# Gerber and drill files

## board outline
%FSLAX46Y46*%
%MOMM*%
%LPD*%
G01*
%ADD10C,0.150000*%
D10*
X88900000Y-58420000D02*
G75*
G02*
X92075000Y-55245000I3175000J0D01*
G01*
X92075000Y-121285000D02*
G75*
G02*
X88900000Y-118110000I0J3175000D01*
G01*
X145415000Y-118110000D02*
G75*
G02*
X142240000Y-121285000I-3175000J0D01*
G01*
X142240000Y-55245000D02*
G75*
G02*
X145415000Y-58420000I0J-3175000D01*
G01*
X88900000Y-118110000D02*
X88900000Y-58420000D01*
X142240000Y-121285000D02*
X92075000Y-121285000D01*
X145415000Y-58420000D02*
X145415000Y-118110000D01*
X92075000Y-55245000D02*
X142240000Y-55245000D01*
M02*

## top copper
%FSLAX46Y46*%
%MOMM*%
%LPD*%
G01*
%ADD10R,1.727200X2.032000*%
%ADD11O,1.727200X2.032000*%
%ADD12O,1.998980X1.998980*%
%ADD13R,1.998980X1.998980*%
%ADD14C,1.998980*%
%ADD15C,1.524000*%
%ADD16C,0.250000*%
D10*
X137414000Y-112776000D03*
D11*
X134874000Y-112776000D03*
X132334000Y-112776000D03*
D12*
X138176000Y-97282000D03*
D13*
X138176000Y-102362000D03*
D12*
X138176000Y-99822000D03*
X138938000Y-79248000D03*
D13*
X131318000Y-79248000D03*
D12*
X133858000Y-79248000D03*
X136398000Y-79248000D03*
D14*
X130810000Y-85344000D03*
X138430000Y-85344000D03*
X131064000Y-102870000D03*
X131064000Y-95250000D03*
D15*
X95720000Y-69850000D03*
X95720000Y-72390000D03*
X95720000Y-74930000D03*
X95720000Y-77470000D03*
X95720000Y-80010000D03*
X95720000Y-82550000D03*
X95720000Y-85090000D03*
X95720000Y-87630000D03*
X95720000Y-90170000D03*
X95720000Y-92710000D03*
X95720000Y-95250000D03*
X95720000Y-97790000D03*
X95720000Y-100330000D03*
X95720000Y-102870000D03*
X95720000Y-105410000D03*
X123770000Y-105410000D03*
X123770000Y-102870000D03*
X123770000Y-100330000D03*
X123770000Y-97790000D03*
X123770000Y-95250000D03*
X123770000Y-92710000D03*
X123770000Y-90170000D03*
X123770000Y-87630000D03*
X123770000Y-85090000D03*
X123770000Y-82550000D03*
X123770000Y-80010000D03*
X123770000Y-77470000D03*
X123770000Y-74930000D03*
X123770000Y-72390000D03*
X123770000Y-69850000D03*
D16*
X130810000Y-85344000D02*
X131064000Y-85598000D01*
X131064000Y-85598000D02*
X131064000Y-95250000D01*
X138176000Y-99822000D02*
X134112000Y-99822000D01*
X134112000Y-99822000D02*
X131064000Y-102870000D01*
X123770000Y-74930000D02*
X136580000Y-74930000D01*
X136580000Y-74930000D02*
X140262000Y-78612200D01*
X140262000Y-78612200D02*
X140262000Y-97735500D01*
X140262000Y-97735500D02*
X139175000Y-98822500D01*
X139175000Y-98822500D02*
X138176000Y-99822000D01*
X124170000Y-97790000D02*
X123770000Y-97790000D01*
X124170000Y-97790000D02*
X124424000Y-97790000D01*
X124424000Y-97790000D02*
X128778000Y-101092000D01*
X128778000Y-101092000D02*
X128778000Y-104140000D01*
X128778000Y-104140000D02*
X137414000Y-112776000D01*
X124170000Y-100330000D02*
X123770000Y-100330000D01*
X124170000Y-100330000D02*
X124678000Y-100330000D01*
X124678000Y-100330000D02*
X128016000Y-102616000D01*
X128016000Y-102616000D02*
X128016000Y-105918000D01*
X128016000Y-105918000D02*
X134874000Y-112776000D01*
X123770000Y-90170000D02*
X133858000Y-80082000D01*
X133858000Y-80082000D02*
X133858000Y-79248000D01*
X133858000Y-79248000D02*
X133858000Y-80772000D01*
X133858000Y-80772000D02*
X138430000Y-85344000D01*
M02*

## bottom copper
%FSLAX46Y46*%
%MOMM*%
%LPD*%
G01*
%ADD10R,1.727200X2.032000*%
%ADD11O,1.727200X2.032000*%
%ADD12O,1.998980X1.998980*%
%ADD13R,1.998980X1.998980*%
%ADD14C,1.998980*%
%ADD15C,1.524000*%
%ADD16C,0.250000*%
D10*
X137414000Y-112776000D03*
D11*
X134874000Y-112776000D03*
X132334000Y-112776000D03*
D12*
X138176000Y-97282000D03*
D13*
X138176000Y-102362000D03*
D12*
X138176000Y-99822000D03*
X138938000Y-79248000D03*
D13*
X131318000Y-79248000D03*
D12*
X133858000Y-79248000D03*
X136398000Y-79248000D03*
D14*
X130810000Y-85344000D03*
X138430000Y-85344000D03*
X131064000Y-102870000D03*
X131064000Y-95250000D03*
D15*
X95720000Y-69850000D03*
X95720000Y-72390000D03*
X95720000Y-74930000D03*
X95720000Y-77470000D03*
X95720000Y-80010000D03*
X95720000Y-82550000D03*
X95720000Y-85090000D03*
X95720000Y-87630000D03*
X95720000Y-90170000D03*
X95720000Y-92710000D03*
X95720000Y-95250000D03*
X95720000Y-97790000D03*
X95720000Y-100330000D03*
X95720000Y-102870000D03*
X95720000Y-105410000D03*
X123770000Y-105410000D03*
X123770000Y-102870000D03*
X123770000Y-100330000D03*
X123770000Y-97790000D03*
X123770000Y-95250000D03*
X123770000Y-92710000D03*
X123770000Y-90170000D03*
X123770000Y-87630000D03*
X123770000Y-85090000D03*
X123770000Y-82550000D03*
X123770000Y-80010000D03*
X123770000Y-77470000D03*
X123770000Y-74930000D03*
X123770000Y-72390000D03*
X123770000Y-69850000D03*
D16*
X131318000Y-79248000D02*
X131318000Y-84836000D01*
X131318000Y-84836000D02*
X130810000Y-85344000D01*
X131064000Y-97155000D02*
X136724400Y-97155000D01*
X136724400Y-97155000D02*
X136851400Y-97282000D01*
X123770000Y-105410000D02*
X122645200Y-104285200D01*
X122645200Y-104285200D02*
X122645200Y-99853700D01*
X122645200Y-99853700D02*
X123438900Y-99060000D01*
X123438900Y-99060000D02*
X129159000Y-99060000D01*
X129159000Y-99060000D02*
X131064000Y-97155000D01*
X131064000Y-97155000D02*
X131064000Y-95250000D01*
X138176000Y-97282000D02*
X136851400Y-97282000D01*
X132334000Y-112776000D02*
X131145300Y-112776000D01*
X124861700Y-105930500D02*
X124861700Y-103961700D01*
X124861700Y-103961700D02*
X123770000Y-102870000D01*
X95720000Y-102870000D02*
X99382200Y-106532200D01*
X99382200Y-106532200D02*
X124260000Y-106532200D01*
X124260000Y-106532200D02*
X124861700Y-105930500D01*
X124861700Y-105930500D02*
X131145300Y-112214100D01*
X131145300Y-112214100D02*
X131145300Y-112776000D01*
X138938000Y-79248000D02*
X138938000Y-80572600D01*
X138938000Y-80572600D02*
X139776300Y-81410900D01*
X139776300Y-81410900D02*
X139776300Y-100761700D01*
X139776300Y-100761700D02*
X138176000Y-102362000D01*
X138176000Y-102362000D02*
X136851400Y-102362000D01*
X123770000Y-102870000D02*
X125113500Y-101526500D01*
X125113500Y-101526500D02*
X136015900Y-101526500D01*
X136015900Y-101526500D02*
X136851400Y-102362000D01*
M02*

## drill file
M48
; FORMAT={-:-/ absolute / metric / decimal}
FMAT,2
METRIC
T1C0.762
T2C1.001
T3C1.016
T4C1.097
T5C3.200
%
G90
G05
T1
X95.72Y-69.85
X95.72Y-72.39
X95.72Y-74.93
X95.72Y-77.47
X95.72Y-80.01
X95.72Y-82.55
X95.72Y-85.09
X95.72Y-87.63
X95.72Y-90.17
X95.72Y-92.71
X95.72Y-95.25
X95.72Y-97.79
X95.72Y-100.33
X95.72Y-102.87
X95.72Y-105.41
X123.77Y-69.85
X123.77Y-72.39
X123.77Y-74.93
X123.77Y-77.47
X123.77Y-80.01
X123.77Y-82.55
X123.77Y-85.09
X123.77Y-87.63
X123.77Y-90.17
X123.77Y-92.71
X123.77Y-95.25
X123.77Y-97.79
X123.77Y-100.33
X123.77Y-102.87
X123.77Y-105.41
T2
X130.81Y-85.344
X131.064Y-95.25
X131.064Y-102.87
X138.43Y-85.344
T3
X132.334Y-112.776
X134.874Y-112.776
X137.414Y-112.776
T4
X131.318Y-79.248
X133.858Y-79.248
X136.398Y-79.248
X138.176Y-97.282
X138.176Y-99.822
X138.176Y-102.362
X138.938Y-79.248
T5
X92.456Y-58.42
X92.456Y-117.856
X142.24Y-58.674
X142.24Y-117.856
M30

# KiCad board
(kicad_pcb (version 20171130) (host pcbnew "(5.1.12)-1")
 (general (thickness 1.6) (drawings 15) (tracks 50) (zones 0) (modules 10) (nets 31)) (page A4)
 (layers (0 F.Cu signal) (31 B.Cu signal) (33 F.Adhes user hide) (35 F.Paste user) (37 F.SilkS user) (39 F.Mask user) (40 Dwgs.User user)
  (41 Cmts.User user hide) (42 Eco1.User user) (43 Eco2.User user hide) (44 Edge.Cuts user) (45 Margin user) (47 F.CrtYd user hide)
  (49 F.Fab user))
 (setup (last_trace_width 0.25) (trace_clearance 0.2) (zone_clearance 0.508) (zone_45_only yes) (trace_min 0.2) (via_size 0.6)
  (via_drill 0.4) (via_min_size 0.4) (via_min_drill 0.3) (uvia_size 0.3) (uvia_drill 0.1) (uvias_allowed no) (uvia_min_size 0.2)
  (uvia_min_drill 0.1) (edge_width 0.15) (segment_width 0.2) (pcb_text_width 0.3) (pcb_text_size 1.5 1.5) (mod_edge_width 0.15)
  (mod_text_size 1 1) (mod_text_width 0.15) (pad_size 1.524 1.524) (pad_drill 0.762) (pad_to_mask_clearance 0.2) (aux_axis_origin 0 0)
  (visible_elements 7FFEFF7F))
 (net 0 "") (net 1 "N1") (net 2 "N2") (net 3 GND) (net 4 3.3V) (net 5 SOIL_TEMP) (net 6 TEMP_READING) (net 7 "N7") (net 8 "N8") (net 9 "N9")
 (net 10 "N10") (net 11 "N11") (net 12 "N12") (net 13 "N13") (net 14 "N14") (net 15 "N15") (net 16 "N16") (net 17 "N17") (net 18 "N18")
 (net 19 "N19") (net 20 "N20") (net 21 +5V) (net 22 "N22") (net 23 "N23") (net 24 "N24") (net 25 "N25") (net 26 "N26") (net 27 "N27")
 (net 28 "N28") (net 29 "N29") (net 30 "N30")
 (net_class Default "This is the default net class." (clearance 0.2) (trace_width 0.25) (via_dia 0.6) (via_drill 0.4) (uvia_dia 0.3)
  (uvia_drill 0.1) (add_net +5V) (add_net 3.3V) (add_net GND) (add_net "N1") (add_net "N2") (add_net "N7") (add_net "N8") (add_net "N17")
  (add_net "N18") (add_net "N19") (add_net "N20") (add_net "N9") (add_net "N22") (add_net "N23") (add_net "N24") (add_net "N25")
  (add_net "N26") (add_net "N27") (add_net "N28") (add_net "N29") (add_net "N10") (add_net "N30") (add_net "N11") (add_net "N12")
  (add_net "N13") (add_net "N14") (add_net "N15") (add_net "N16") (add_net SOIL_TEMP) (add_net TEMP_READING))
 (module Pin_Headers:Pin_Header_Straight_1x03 (layer F.Cu) (at 137.414 112.776 270)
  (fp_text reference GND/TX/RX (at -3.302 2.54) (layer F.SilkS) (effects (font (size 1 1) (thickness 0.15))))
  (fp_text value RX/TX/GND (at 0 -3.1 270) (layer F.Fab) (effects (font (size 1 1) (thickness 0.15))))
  (pad 1 thru_hole rect (at 0 0 270) (size 2.032 1.7272) (drill 1.016) (layers *.Cu *.Mask F.SilkS) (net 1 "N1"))
  (pad 2 thru_hole oval (at 0 2.54 270) (size 2.032 1.7272) (drill 1.016) (layers *.Cu *.Mask F.SilkS) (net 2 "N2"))
  (pad 3 thru_hole oval (at 0 5.08 270) (size 2.032 1.7272) (drill 1.016) (layers *.Cu *.Mask F.SilkS) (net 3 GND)))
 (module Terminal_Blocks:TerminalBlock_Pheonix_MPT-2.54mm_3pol (layer F.Cu) (at 138.176 102.362 90)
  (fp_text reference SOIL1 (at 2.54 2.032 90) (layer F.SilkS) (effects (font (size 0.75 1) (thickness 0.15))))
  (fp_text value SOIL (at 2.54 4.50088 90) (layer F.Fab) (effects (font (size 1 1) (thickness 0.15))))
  (pad 3 thru_hole oval (at 5.08 0 90) (size 1.99898 1.99898) (drill 1.09728) (layers *.Cu *.Mask F.SilkS) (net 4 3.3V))
  (pad 1 thru_hole rect (at 0 0 90) (size 1.99898 1.99898) (drill 1.09728) (layers *.Cu *.Mask F.SilkS) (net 3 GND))
  (pad 2 thru_hole oval (at 2.54 0 90) (size 1.99898 1.99898) (drill 1.09728) (layers *.Cu *.Mask F.SilkS) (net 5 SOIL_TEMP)))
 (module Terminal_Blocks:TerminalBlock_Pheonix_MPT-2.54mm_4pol (layer F.Cu) (at 131.318 79.248)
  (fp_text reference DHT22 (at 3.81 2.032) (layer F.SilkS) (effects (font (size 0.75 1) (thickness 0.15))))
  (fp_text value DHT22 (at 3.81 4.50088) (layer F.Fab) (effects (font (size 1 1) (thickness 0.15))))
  (pad 4 thru_hole oval (at 7.62 0 180) (size 1.99898 1.99898) (drill 1.09728) (layers *.Cu *.Mask F.SilkS) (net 3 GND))
  (pad 1 thru_hole rect (at 0 0 180) (size 1.99898 1.99898) (drill 1.09728) (layers *.Cu *.Mask F.SilkS) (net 4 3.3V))
  (pad 2 thru_hole oval (at 2.54 0 180) (size 1.99898 1.99898) (drill 1.09728) (layers *.Cu *.Mask F.SilkS) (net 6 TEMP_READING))
  (pad 3 thru_hole oval (at 5.08 0 180) (size 1.99898 1.99898) (drill 1.09728) (layers *.Cu *.Mask F.SilkS) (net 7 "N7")))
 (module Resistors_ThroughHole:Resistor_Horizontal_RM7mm (layer F.Cu) (at 130.81 85.344)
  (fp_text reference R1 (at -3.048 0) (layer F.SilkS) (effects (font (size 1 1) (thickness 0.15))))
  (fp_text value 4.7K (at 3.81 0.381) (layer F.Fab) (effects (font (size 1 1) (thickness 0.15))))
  (pad 1 thru_hole circle (at 0 0) (size 1.99898 1.99898) (drill 1.00076) (layers *.Cu *.SilkS *.Mask) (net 4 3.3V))
  (pad 2 thru_hole circle (at 7.62 0) (size 1.99898 1.99898) (drill 1.00076) (layers *.Cu *.SilkS *.Mask) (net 6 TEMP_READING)))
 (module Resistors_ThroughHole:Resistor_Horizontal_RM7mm (layer F.Cu) (at 131.064 102.87 90)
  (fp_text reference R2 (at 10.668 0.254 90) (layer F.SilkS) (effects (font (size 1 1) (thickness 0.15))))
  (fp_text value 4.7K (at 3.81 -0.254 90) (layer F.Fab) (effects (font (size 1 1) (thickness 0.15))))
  (pad 1 thru_hole circle (at 0 0 90) (size 1.99898 1.99898) (drill 1.00076) (layers *.Cu *.SilkS *.Mask) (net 5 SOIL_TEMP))
  (pad 2 thru_hole circle (at 7.62 0 90) (size 1.99898 1.99898) (drill 1.00076) (layers *.Cu *.SilkS *.Mask) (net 4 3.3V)))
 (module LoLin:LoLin (layer F.Cu) (at 93.98 59.69)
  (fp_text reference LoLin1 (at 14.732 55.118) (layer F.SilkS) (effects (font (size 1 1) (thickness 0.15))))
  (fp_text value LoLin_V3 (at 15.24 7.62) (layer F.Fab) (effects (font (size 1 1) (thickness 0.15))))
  (pad 1 thru_hole circle (at 1.74 10.16) (size 1.524 1.524) (drill 0.762) (layers *.Cu *.Mask F.SilkS) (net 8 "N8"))
  (pad 2 thru_hole circle (at 1.74 12.7) (size 1.524 1.524) (drill 0.762) (layers *.Cu *.Mask F.SilkS) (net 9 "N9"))
  (pad 3 thru_hole circle (at 1.74 15.24) (size 1.524 1.524) (drill 0.762) (layers *.Cu *.Mask F.SilkS) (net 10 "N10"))
  (pad 4 thru_hole circle (at 1.74 17.78) (size 1.524 1.524) (drill 0.762) (layers *.Cu *.Mask F.SilkS) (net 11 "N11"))
  (pad 5 thru_hole circle (at 1.74 20.32) (size 1.524 1.524) (drill 0.762) (layers *.Cu *.Mask F.SilkS) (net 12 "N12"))
  (pad 6 thru_hole circle (at 1.74 22.86) (size 1.524 1.524) (drill 0.762) (layers *.Cu *.Mask F.SilkS) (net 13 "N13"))
  (pad 7 thru_hole circle (at 1.74 25.4) (size 1.524 1.524) (drill 0.762) (layers *.Cu *.Mask F.SilkS) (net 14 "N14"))
  (pad 8 thru_hole circle (at 1.74 27.94) (size 1.524 1.524) (drill 0.762) (layers *.Cu *.Mask F.SilkS) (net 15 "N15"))
  (pad 9 thru_hole circle (at 1.74 30.48) (size 1.524 1.524) (drill 0.762) (layers *.Cu *.Mask F.SilkS) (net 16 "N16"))
  (pad 10 thru_hole circle (at 1.74 33.02) (size 1.524 1.524) (drill 0.762) (layers *.Cu *.Mask F.SilkS) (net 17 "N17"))
  (pad 11 thru_hole circle (at 1.74 35.56) (size 1.524 1.524) (drill 0.762) (layers *.Cu *.Mask F.SilkS) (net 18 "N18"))
  (pad 12 thru_hole circle (at 1.74 38.1) (size 1.524 1.524) (drill 0.762) (layers *.Cu *.Mask F.SilkS) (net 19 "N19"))
  (pad 13 thru_hole circle (at 1.74 40.64) (size 1.524 1.524) (drill 0.762) (layers *.Cu *.Mask F.SilkS) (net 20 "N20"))
  (pad 14 thru_hole circle (at 1.74 43.18) (size 1.524 1.524) (drill 0.762) (layers *.Cu *.Mask F.SilkS) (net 3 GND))
  (pad 15 thru_hole circle (at 1.74 45.72) (size 1.524 1.524) (drill 0.762) (layers *.Cu *.Mask F.SilkS) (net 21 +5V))
  (pad 16 thru_hole circle (at 29.79 45.72) (size 1.524 1.524) (drill 0.762) (layers *.Cu *.Mask F.SilkS) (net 4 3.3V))
  (pad 17 thru_hole circle (at 29.79 43.18) (size 1.524 1.524) (drill 0.762) (layers *.Cu *.Mask F.SilkS) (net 3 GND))
  (pad 18 thru_hole circle (at 29.79 40.64) (size 1.524 1.524) (drill 0.762) (layers *.Cu *.Mask F.SilkS) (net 2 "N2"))
  (pad 19 thru_hole circle (at 29.79 38.1) (size 1.524 1.524) (drill 0.762) (layers *.Cu *.Mask F.SilkS) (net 1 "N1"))
  (pad 20 thru_hole circle (at 29.79 35.56) (size 1.524 1.524) (drill 0.762) (layers *.Cu *.Mask F.SilkS) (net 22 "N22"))
  (pad 21 thru_hole circle (at 29.79 33.02) (size 1.524 1.524) (drill 0.762) (layers *.Cu *.Mask F.SilkS) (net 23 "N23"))
  (pad 22 thru_hole circle (at 29.79 30.48) (size 1.524 1.524) (drill 0.762) (layers *.Cu *.Mask F.SilkS) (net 6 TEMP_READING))
  (pad 23 thru_hole circle (at 29.79 27.94) (size 1.524 1.524) (drill 0.762) (layers *.Cu *.Mask F.SilkS) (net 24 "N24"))
  (pad 24 thru_hole circle (at 29.79 25.4) (size 1.524 1.524) (drill 0.762) (layers *.Cu *.Mask F.SilkS) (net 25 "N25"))
  (pad 25 thru_hole circle (at 29.79 22.86) (size 1.524 1.524) (drill 0.762) (layers *.Cu *.Mask F.SilkS) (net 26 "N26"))
  (pad 26 thru_hole circle (at 29.79 20.32) (size 1.524 1.524) (drill 0.762) (layers *.Cu *.Mask F.SilkS) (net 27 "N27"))
  (pad 27 thru_hole circle (at 29.79 17.78) (size 1.524 1.524) (drill 0.762) (layers *.Cu *.Mask F.SilkS) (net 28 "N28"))
  (pad 28 thru_hole circle (at 29.79 15.24) (size 1.524 1.524) (drill 0.762) (layers *.Cu *.Mask F.SilkS) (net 5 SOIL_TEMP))
  (pad 29 thru_hole circle (at 29.79 12.7) (size 1.524 1.524) (drill 0.762) (layers *.Cu *.Mask F.SilkS) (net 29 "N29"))
  (pad 30 thru_hole circle (at 29.79 10.16) (size 1.524 1.524) (drill 0.762) (layers *.Cu *.Mask F.SilkS) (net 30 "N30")))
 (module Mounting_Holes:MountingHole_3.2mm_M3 (layer F.Cu) (at 93.472 58.42)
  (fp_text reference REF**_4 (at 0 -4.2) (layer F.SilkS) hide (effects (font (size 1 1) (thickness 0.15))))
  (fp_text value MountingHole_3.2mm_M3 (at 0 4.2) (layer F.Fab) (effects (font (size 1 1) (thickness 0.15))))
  (pad 1 np_thru_hole circle (at -1.016 0) (size 3.2 3.2) (drill 3.2) (layers *.Cu *.Mask F.SilkS)))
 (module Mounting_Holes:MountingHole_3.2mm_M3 (layer F.Cu) (at 142.24 58.674)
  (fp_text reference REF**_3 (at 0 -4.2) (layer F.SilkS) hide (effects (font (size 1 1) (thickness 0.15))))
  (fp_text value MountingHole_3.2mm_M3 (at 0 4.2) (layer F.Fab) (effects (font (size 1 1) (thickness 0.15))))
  (pad 1 np_thru_hole circle (at 0 0) (size 3.2 3.2) (drill 3.2) (layers *.Cu *.Mask F.SilkS)))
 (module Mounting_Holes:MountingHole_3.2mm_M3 (layer F.Cu) (at 142.24 117.856)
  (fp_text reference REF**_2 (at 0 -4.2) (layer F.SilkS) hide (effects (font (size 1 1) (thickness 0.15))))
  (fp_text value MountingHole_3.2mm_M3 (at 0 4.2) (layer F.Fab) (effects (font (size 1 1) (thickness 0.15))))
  (pad 1 np_thru_hole circle (at 0 0) (size 3.2 3.2) (drill 3.2) (layers *.Cu *.Mask F.SilkS)))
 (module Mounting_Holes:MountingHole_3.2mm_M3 (layer F.Cu) (at 93.472 117.856)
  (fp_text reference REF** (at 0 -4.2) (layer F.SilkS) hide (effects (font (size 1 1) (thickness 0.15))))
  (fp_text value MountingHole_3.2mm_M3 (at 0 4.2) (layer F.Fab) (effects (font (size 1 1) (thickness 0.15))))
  (pad 1 np_thru_hole circle (at -1.016 0) (size 3.2 3.2) (drill 3.2) (layers *.Cu *.Mask F.SilkS)))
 (gr_arc (start 92.075 58.42) (end 88.9 58.42) (angle 90) (layer Edge.Cuts) (width 0.15))
 (gr_arc (start 92.075 118.11) (end 92.075 121.285) (angle 90) (layer Edge.Cuts) (width 0.15))
 (gr_arc (start 142.24 118.11) (end 145.415 118.11) (angle 90) (layer Edge.Cuts) (width 0.15))
 (gr_arc (start 142.24 58.42) (end 142.24 55.245) (angle 90) (layer Edge.Cuts) (width 0.15))
 (gr_line (start 88.9 118.11) (end 88.9 58.42) (angle 90) (layer Edge.Cuts) (width 0.15))
 (gr_line (start 142.24 121.285) (end 92.075 121.285) (angle 90) (layer Edge.Cuts) (width 0.15))
 (gr_line (start 145.415 58.42) (end 145.415 118.11) (angle 90) (layer Edge.Cuts) (width 0.15))
 (gr_line (start 92.075 55.245) (end 142.24 55.245) (angle 90) (layer Edge.Cuts) (width 0.15))
 (segment (start 131.318 79.248) (end 131.318 84.836) (width 0.25) (layer B.Cu) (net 4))
 (segment (start 131.318 84.836) (end 130.81 85.344) (width 0.25) (layer B.Cu) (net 4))
 (segment (start 130.81 85.344) (end 131.064 85.598) (width 0.25) (layer F.Cu) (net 4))
 (segment (start 131.064 85.598) (end 131.064 95.25) (width 0.25) (layer F.Cu) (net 4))
 (segment (start 131.064 97.155) (end 136.7244 97.155) (width 0.25) (layer B.Cu) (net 4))
 (segment (start 136.7244 97.155) (end 136.8514 97.282) (width 0.25) (layer B.Cu) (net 4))
 (segment (start 123.77 105.41) (end 122.6452 104.2852) (width 0.25) (layer B.Cu) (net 4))
 (segment (start 122.6452 104.2852) (end 122.6452 99.8537) (width 0.25) (layer B.Cu) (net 4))
 (segment (start 122.6452 99.8537) (end 123.4389 99.06) (width 0.25) (layer B.Cu) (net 4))
 (segment (start 123.4389 99.06) (end 129.159 99.06) (width 0.25) (layer B.Cu) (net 4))
 (segment (start 129.159 99.06) (end 131.064 97.155) (width 0.25) (layer B.Cu) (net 4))
 (segment (start 131.064 97.155) (end 131.064 95.25) (width 0.25) (layer B.Cu) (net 4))
 (segment (start 138.176 97.282) (end 136.8514 97.282) (width 0.25) (layer B.Cu) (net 4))
 (segment (start 132.334 112.776) (end 131.1453 112.776) (width 0.25) (layer B.Cu) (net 3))
 (segment (start 124.8617 105.9305) (end 124.8617 103.9617) (width 0.25) (layer B.Cu) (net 3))
 (segment (start 124.8617 103.9617) (end 123.77 102.87) (width 0.25) (layer B.Cu) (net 3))
 (segment (start 95.72 102.87) (end 99.3822 106.5322) (width 0.25) (layer B.Cu) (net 3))
 (segment (start 99.3822 106.5322) (end 124.26 106.5322) (width 0.25) (layer B.Cu) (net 3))
 (segment (start 124.26 106.5322) (end 124.8617 105.9305) (width 0.25) (layer B.Cu) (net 3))
 (segment (start 124.8617 105.9305) (end 131.1453 112.2141) (width 0.25) (layer B.Cu) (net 3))
 (segment (start 131.1453 112.2141) (end 131.1453 112.776) (width 0.25) (layer B.Cu) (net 3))
 (segment (start 138.938 79.248) (end 138.938 80.5726) (width 0.25) (layer B.Cu) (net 3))
 (segment (start 138.938 80.5726) (end 139.7763 81.4109) (width 0.25) (layer B.Cu) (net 3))
 (segment (start 139.7763 81.4109) (end 139.7763 100.7617) (width 0.25) (layer B.Cu) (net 3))
 (segment (start 139.7763 100.7617) (end 138.176 102.362) (width 0.25) (layer B.Cu) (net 3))
 (segment (start 138.176 102.362) (end 136.8514 102.362) (width 0.25) (layer B.Cu) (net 3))
 (segment (start 123.77 102.87) (end 125.1135 101.5265) (width 0.25) (layer B.Cu) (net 3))
 (segment (start 125.1135 101.5265) (end 136.0159 101.5265) (width 0.25) (layer B.Cu) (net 3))
 (segment (start 136.0159 101.5265) (end 136.8514 102.362) (width 0.25) (layer B.Cu) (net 3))
 (segment (start 138.176 99.822) (end 134.112 99.822) (width 0.25) (layer F.Cu) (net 5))
 (segment (start 134.112 99.822) (end 131.064 102.87) (width 0.25) (layer F.Cu) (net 5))
 (segment (start 123.77 74.93) (end 136.58 74.93) (width 0.25) (layer F.Cu) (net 5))
 (segment (start 136.58 74.93) (end 140.262 78.6122) (width 0.25) (layer F.Cu) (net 5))
 (segment (start 140.262 78.6122) (end 140.262 97.7355) (width 0.25) (layer F.Cu) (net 5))
 (segment (start 140.262 97.7355) (end 139.175 98.8225) (width 0.25) (layer F.Cu) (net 5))
 (segment (start 139.175 98.8225) (end 138.176 99.822) (width 0.25) (layer F.Cu) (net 5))
 (segment (start 124.17 97.79) (end 123.77 97.79) (width 0.25) (layer F.Cu) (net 1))
 (segment (start 124.17 97.79) (end 124.424 97.79) (width 0.25) (layer F.Cu) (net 1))
 (segment (start 124.424 97.79) (end 128.778 101.092) (width 0.25) (layer F.Cu) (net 1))
 (segment (start 128.778 101.092) (end 128.778 104.14) (width 0.25) (layer F.Cu) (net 1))
 (segment (start 128.778 104.14) (end 137.414 112.776) (width 0.25) (layer F.Cu) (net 1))
 (segment (start 124.17 100.33) (end 123.77 100.33) (width 0.25) (layer F.Cu) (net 2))
 (segment (start 124.17 100.33) (end 124.678 100.33) (width 0.25) (layer F.Cu) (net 2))
 (segment (start 124.678 100.33) (end 128.016 102.616) (width 0.25) (layer F.Cu) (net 2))
 (segment (start 128.016 102.616) (end 128.016 105.918) (width 0.25) (layer F.Cu) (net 2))
 (segment (start 128.016 105.918) (end 134.874 112.776) (width 0.25) (layer F.Cu) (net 2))
 (segment (start 123.77 90.17) (end 133.858 80.082) (width 0.25) (layer F.Cu) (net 6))
 (segment (start 133.858 80.082) (end 133.858 79.248) (width 0.25) (layer F.Cu) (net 6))
 (segment (start 133.858 79.248) (end 133.858 80.772) (width 0.25) (layer F.Cu) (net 6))
 (segment (start 133.858 80.772) (end 138.43 85.344) (width 0.25) (layer F.Cu) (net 6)))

